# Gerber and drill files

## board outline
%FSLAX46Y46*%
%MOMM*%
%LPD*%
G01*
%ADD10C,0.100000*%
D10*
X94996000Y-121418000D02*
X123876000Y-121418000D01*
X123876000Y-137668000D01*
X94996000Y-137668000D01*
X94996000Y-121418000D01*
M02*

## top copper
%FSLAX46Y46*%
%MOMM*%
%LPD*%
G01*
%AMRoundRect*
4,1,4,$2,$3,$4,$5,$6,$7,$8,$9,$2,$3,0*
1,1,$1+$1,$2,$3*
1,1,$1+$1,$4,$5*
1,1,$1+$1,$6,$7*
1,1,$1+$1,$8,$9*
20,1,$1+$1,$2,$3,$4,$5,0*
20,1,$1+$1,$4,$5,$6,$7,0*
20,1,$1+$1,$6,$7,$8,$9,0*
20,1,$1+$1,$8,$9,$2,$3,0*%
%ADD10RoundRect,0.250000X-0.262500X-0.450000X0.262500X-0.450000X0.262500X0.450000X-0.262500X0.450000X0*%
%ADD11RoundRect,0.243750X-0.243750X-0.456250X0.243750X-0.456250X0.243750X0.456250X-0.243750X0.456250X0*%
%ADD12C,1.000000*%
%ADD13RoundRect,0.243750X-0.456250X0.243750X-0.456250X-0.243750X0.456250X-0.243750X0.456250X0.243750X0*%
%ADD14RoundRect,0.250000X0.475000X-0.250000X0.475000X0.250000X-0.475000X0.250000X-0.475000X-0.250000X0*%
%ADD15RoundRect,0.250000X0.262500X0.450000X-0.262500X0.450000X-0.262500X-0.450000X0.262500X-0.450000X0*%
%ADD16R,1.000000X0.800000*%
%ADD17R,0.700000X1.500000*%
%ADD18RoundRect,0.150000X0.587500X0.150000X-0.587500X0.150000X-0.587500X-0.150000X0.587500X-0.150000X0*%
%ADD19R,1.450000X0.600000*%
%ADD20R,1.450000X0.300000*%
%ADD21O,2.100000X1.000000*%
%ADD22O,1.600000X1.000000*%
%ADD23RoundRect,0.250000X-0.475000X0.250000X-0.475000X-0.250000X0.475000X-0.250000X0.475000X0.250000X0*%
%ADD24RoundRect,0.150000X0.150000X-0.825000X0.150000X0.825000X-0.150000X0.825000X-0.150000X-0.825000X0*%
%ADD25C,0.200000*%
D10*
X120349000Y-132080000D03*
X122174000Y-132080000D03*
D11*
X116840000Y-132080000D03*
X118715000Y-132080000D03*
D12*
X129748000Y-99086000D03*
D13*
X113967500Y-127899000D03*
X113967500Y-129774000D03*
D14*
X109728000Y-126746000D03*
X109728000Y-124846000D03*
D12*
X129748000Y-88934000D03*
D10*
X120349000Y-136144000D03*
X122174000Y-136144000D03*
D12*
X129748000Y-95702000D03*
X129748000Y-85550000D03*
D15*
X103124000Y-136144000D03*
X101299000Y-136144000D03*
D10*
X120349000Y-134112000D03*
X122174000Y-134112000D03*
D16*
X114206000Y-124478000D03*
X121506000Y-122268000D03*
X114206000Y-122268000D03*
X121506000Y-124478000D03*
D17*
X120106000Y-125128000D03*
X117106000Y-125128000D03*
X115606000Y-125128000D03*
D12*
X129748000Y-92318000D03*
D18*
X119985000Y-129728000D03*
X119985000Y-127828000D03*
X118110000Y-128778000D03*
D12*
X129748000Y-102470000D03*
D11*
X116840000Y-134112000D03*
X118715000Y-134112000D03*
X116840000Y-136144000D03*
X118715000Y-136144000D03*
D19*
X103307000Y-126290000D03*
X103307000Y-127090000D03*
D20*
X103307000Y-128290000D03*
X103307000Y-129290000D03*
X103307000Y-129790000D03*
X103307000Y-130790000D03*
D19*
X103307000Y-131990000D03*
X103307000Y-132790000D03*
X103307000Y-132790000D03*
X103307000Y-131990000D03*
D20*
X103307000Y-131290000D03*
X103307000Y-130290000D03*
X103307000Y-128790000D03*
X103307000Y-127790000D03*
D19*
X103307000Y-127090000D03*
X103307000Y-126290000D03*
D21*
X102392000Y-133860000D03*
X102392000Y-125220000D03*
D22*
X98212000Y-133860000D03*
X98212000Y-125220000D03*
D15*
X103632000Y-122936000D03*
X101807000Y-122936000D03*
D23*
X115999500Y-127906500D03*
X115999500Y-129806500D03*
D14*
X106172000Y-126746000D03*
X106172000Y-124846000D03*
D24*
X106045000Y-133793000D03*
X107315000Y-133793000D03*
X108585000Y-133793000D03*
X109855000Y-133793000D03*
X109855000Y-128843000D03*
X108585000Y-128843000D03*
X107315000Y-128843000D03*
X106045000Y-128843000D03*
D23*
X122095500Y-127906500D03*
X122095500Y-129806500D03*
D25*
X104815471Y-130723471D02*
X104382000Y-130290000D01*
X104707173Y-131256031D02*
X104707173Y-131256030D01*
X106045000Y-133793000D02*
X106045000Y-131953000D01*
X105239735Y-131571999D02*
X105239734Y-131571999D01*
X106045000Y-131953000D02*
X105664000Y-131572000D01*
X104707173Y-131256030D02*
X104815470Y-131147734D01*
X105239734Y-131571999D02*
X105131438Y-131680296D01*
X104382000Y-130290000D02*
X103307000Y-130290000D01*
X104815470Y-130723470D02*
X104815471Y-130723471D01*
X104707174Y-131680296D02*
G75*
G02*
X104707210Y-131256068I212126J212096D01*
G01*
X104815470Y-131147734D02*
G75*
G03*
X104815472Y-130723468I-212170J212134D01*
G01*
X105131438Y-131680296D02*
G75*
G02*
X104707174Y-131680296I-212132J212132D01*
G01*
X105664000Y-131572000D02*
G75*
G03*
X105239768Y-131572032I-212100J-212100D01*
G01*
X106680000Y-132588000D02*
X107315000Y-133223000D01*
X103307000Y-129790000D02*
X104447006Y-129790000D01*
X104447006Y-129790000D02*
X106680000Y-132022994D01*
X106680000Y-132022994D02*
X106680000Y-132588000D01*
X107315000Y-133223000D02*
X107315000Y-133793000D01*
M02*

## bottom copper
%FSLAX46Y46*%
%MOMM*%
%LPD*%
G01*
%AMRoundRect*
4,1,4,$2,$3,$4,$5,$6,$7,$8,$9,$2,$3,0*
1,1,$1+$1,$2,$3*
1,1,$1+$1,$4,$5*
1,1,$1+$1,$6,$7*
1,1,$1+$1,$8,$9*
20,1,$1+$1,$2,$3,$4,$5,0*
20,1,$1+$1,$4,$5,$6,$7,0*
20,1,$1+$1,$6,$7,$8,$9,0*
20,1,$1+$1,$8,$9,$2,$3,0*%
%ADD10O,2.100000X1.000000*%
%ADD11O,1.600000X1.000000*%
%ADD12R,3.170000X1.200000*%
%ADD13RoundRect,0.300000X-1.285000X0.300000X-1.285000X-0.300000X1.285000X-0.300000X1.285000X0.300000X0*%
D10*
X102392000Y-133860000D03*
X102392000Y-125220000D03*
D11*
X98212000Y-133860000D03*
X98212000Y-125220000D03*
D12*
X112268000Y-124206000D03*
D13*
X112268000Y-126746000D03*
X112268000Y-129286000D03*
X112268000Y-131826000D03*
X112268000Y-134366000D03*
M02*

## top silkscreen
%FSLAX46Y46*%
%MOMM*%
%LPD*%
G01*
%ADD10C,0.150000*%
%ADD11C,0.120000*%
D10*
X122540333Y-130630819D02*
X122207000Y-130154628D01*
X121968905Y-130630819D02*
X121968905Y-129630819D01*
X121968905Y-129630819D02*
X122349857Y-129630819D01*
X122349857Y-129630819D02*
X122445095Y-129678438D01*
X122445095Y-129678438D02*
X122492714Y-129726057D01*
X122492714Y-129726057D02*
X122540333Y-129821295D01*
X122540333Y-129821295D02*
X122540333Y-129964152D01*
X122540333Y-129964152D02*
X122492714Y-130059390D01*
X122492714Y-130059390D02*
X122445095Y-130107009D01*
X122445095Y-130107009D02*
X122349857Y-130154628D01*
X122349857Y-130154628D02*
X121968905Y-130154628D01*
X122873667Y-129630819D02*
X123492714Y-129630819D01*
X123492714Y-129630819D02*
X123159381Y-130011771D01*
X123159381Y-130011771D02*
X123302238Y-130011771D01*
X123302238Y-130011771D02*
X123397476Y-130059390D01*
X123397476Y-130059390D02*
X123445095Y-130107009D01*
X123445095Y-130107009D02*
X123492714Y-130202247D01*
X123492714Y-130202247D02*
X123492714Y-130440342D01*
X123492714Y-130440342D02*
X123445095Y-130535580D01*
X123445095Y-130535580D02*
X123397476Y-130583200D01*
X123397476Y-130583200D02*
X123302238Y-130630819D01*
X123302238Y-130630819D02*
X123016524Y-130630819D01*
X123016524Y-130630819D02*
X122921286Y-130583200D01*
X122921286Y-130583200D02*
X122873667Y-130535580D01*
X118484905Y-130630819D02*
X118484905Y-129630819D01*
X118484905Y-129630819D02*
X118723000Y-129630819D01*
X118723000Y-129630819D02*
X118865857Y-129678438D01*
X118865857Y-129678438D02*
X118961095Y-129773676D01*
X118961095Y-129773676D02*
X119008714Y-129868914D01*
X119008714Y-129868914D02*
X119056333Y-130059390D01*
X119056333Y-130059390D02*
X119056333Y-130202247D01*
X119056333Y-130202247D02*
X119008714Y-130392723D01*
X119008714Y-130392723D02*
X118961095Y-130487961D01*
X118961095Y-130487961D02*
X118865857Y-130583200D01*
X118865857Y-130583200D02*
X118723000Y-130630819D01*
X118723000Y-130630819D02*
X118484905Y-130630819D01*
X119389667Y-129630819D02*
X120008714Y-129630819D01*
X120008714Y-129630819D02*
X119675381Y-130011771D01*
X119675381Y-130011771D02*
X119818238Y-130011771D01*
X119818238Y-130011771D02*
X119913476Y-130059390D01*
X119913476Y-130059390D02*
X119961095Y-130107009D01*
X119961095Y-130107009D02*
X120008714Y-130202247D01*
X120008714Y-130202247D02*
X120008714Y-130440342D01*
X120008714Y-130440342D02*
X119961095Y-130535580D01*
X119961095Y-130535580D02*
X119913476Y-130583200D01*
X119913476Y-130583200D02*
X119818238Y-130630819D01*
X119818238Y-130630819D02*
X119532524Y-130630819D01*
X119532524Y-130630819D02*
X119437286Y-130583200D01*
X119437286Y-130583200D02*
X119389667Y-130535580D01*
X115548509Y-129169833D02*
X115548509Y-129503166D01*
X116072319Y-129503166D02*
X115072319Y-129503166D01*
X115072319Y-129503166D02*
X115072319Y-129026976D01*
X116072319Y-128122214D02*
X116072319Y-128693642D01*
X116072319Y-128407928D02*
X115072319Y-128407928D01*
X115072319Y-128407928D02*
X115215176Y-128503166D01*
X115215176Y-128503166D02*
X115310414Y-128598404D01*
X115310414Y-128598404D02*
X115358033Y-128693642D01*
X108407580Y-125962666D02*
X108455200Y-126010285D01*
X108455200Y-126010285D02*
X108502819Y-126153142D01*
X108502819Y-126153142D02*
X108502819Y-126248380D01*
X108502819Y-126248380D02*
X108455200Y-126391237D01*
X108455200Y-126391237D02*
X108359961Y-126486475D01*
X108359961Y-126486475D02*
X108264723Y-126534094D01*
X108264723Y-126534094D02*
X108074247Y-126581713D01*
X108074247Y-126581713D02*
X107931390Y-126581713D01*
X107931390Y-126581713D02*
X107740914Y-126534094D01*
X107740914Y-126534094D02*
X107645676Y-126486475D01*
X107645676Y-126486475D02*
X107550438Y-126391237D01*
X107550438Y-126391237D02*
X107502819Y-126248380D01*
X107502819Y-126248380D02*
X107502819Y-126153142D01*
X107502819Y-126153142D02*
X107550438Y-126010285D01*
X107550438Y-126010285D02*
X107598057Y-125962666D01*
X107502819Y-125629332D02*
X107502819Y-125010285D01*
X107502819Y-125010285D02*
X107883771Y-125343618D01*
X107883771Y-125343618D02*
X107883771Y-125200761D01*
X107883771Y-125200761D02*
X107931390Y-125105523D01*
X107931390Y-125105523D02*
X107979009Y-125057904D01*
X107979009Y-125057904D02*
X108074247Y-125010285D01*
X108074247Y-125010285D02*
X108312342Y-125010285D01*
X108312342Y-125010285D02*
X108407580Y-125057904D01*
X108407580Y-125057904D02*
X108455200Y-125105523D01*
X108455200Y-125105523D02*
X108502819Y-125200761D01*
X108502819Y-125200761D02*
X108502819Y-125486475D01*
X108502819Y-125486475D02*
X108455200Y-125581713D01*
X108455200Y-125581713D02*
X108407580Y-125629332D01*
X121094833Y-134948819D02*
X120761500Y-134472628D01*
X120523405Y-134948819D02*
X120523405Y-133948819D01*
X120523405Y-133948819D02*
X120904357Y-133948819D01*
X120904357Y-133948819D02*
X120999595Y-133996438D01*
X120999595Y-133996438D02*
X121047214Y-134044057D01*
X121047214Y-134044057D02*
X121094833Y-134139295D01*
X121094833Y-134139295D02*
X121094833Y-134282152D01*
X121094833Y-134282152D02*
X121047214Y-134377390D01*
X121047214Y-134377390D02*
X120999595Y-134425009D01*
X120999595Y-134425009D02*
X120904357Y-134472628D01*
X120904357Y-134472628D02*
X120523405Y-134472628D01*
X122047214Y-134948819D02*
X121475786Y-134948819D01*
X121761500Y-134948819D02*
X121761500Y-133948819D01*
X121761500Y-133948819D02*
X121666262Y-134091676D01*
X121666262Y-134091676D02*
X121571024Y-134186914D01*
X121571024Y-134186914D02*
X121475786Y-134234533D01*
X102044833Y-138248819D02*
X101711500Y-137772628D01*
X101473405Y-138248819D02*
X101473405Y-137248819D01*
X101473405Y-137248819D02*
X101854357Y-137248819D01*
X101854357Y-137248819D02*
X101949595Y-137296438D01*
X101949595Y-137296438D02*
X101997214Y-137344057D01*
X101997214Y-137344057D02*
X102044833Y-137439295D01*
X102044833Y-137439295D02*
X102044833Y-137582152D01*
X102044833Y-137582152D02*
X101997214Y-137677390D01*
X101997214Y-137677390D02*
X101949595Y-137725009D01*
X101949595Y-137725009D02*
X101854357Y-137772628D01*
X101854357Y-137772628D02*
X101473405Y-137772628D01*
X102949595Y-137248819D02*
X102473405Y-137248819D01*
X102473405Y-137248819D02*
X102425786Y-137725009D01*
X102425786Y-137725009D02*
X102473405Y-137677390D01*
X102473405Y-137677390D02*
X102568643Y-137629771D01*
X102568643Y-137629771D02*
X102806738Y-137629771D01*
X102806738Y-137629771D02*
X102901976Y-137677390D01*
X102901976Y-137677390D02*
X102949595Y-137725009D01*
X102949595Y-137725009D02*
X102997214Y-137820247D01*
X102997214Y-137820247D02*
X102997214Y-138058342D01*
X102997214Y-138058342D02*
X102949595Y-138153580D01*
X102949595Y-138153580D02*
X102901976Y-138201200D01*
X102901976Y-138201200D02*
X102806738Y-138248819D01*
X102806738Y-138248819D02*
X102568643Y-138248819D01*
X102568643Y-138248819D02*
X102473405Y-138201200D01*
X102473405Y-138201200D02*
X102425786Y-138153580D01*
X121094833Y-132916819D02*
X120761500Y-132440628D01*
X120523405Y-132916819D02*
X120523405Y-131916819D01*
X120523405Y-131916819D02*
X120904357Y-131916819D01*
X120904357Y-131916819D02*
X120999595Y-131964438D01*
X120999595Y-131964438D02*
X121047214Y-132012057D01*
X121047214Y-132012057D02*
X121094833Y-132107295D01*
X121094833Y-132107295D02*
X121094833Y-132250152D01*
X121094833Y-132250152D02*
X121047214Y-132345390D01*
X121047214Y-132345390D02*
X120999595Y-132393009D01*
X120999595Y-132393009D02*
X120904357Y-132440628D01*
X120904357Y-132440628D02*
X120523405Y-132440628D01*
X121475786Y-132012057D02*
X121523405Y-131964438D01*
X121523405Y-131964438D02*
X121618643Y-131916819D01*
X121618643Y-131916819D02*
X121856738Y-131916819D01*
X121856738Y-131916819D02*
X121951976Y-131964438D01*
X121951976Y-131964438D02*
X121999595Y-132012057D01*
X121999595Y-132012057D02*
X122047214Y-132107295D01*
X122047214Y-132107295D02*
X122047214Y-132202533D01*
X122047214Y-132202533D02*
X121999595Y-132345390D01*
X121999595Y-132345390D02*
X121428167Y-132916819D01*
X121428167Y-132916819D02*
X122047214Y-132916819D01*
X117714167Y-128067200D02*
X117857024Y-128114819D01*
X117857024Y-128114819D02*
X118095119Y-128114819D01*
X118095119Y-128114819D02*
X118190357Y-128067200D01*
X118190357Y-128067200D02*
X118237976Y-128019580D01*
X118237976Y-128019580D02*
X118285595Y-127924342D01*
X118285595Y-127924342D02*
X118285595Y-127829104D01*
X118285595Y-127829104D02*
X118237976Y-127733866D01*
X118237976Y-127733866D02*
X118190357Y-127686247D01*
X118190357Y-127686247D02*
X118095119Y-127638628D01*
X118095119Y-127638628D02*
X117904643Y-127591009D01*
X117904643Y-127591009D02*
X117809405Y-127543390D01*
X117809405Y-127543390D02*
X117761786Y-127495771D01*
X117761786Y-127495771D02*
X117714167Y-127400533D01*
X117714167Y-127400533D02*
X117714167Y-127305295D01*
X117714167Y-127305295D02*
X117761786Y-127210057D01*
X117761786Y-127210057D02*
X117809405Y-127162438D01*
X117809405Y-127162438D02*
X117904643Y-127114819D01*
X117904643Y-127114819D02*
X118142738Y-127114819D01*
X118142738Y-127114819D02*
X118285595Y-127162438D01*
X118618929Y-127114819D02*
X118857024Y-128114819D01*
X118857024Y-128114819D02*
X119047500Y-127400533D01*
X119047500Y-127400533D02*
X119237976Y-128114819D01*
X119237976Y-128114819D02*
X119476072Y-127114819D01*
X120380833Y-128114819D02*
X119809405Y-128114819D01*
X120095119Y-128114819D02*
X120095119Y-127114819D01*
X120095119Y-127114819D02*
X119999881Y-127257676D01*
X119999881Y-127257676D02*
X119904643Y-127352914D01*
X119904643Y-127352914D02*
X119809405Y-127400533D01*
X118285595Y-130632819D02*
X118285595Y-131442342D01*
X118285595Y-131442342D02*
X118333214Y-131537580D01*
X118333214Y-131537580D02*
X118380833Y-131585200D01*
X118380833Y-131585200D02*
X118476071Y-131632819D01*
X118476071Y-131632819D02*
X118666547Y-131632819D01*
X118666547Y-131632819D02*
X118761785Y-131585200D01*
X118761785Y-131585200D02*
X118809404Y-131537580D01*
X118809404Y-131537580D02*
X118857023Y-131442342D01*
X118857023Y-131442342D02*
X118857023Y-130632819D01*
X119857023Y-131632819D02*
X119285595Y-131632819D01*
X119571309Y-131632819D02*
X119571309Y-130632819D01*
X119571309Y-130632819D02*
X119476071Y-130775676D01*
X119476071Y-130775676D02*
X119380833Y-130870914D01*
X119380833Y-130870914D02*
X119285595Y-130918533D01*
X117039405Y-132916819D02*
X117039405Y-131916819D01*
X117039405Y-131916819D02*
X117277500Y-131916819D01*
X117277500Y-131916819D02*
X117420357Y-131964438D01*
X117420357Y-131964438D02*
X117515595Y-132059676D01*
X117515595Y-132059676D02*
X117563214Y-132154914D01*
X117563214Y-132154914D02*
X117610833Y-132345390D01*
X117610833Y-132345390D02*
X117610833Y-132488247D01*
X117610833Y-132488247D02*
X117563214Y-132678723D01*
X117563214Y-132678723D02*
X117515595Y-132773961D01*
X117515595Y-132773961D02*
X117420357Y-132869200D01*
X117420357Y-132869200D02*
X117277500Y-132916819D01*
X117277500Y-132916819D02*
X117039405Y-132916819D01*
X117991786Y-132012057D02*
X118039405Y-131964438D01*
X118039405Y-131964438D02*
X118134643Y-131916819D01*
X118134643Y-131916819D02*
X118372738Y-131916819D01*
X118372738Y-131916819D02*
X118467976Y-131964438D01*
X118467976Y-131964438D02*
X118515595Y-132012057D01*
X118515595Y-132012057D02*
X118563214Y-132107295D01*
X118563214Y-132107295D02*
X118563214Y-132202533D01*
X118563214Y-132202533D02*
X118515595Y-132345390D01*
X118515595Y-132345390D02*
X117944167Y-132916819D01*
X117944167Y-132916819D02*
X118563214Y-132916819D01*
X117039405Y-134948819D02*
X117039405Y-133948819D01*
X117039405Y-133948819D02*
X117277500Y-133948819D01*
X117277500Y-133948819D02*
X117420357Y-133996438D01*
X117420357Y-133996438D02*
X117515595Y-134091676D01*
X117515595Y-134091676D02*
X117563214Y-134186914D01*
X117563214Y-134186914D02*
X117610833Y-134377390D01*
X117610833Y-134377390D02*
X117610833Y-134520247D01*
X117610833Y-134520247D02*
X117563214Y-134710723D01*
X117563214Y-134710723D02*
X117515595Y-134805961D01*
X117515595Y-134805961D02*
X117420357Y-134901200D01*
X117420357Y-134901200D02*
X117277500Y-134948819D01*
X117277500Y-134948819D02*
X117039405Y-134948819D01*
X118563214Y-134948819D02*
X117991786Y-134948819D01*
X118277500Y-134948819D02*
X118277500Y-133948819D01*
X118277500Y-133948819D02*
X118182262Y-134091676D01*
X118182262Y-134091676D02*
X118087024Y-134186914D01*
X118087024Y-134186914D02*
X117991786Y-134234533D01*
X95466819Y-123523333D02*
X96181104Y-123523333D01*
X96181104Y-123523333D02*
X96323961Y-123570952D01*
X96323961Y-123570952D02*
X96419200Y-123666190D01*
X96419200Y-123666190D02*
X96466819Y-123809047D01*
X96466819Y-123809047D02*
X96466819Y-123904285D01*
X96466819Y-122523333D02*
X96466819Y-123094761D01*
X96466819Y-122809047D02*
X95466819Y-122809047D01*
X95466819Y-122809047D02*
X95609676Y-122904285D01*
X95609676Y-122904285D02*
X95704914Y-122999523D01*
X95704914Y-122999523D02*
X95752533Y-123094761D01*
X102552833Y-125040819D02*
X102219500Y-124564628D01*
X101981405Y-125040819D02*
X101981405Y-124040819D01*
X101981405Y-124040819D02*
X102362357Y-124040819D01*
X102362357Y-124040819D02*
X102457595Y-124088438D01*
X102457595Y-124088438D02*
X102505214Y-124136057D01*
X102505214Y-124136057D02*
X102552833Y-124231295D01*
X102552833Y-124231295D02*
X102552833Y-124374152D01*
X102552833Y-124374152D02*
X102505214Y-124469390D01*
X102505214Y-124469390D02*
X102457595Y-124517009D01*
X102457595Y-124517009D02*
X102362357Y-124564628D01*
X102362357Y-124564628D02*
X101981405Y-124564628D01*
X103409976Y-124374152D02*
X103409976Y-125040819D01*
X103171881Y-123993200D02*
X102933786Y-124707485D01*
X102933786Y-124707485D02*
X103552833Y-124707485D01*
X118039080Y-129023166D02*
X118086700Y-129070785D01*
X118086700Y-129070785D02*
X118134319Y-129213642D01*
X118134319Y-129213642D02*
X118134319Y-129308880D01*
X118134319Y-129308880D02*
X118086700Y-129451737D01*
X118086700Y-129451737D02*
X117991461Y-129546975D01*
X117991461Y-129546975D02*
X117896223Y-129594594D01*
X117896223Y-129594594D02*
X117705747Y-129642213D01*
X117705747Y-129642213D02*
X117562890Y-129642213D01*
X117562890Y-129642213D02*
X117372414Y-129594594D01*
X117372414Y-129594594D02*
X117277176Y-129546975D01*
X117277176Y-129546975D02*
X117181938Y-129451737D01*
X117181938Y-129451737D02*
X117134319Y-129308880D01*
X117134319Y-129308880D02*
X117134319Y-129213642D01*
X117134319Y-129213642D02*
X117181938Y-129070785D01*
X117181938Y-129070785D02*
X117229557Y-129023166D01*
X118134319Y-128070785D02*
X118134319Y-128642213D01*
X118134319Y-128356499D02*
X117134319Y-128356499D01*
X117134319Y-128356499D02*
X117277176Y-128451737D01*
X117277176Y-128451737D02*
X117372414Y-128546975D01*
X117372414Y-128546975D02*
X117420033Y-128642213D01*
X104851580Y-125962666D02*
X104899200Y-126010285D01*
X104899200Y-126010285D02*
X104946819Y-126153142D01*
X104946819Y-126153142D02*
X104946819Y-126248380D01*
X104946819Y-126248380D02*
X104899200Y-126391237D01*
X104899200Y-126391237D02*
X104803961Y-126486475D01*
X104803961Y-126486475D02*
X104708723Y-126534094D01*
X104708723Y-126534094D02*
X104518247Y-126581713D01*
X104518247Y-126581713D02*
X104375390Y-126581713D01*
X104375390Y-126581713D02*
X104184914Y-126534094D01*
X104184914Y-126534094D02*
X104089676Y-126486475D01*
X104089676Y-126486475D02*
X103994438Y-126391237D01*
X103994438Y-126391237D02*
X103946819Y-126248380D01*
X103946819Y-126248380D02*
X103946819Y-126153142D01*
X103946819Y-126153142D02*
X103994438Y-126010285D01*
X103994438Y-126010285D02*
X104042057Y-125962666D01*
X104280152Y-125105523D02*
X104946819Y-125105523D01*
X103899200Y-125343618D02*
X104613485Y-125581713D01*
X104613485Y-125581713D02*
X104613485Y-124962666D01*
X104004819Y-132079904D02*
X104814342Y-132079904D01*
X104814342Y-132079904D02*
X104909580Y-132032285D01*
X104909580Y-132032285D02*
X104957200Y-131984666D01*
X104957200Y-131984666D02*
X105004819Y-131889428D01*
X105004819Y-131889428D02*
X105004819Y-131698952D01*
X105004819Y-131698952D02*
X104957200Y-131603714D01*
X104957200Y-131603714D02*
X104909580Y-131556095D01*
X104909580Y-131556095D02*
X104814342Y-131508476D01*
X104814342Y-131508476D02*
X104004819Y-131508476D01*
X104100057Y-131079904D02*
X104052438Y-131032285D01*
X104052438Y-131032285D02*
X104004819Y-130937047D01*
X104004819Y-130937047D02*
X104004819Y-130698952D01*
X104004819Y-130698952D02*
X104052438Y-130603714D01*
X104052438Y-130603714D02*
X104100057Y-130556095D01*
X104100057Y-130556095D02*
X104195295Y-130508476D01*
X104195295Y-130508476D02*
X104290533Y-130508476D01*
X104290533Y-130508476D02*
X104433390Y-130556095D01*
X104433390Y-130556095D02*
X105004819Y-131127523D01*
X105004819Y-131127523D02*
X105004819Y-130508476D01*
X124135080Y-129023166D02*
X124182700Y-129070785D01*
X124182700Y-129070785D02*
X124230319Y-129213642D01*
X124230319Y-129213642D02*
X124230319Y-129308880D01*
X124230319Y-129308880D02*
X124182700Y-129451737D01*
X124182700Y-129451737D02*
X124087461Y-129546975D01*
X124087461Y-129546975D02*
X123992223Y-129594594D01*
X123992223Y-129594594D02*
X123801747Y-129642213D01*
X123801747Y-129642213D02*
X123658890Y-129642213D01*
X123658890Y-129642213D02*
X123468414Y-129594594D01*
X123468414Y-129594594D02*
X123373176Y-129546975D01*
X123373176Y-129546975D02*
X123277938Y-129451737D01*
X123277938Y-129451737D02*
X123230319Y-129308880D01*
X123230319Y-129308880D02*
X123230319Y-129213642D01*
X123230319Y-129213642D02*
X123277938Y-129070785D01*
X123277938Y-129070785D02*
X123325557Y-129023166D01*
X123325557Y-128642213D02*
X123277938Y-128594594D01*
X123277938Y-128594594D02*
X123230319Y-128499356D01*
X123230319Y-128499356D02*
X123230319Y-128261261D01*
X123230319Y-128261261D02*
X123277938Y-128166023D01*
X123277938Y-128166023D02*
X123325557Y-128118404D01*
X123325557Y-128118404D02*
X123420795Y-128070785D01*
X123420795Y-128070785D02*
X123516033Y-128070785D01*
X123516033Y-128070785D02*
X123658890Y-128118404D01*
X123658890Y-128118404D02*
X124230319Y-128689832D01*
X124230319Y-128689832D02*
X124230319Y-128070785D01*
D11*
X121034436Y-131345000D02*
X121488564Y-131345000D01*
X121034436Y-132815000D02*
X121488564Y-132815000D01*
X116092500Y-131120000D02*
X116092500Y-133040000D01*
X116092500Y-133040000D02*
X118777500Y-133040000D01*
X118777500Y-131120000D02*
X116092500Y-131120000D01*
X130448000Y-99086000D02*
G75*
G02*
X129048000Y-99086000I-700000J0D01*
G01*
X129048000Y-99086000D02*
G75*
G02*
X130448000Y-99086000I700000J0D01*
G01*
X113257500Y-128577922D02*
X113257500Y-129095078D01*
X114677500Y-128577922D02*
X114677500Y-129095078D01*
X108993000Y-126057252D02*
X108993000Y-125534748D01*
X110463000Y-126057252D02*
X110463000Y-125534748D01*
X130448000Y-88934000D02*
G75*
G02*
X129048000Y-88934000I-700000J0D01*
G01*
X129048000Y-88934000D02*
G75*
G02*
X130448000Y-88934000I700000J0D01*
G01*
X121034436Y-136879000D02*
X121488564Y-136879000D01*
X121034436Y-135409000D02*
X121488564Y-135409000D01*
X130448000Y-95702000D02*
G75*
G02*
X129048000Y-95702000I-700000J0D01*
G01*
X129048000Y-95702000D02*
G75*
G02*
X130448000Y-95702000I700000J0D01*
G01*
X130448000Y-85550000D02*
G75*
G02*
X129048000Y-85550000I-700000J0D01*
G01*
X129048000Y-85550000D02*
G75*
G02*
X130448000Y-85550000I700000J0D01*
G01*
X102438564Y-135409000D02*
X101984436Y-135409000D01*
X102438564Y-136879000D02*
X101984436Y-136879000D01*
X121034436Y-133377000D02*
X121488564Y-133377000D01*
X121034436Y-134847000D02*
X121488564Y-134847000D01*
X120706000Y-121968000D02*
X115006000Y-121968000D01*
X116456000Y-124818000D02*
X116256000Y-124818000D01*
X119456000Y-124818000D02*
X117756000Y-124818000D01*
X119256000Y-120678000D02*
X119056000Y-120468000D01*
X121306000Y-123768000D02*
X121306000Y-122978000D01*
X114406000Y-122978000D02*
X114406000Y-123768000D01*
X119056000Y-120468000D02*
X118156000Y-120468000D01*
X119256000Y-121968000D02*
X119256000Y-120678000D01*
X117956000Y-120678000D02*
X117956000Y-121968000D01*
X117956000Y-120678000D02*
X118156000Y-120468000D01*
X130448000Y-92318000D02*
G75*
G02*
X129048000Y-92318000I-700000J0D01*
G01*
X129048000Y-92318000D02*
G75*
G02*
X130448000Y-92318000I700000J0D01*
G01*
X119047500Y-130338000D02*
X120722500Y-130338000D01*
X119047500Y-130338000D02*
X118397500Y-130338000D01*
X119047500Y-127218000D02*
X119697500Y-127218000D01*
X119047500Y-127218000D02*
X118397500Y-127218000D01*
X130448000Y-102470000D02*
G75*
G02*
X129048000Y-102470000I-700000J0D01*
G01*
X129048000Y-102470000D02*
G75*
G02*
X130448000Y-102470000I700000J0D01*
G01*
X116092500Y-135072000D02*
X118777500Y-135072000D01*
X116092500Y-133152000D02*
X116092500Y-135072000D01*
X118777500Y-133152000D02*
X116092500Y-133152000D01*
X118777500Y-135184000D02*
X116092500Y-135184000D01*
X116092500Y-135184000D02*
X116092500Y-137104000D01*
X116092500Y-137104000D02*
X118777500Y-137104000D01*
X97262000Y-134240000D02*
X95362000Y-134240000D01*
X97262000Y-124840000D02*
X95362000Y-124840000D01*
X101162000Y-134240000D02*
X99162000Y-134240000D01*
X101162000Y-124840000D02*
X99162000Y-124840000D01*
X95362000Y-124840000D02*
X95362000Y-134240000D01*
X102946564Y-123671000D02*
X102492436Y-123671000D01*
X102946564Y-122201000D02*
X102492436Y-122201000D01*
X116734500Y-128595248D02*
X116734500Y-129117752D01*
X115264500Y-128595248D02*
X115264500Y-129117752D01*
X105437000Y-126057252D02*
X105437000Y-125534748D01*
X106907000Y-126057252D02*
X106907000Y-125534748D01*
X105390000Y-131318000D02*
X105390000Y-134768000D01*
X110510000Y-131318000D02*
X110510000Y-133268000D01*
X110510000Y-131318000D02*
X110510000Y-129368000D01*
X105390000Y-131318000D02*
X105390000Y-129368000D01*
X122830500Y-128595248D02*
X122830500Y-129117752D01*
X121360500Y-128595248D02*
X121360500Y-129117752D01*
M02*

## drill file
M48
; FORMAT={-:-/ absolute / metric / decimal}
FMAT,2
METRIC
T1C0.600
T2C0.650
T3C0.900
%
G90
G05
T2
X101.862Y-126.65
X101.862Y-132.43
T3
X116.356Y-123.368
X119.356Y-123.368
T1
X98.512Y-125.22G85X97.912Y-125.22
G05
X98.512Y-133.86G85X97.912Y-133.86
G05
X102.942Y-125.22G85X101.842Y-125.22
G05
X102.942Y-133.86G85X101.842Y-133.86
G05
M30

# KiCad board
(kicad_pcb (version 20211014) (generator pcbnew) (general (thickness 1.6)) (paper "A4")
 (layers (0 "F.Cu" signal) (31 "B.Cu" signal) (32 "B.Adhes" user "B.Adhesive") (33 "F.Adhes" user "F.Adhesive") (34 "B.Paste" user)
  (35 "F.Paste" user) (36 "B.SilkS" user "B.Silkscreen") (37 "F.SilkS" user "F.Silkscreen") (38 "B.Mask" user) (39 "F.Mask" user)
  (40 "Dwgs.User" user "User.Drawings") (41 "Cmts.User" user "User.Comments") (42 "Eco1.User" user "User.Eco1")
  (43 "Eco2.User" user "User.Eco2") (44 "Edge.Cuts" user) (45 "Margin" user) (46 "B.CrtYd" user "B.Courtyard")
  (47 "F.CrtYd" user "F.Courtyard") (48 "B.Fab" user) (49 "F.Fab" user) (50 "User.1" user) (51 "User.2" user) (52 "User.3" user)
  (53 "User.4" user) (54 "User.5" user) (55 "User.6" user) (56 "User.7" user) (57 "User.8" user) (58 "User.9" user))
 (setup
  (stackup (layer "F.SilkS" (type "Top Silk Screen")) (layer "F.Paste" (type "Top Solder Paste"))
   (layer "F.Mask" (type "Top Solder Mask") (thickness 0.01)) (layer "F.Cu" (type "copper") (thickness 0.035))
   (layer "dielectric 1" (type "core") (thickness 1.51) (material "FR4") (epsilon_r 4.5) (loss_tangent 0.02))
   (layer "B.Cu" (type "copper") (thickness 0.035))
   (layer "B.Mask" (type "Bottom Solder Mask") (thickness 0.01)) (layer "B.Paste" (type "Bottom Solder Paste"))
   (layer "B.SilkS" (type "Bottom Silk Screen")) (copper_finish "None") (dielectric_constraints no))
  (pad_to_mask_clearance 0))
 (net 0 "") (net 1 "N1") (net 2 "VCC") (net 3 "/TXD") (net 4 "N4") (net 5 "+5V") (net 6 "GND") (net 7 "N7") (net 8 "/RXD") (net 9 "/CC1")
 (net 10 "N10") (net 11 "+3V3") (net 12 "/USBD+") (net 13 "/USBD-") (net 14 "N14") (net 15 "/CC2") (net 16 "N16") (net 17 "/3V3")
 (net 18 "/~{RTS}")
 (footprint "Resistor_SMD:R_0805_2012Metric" (layer "F.Cu") (at 121.2615 132.08)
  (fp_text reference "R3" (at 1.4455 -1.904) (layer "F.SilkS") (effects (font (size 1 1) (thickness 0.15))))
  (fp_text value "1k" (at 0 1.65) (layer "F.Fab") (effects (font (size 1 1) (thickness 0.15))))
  (fp_line (start -0.227064 -0.735) (end 0.227064 -0.735) (layer "F.SilkS") (width 0.12))
  (fp_line (start -0.227064 0.735) (end 0.227064 0.735) (layer "F.SilkS") (width 0.12))
  (pad "1" smd roundrect (at -0.9125 0) (size 1.025 1.4) (layers "F.Cu" "F.Paste" "F.Mask") (roundrect_rratio 0.243902) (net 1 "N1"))
  (pad "2" smd roundrect (at 0.9125 0) (size 1.025 1.4) (layers "F.Cu" "F.Paste" "F.Mask") (roundrect_rratio 0.243902) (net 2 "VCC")))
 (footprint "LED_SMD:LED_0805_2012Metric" (layer "F.Cu") (at 117.7775 132.08)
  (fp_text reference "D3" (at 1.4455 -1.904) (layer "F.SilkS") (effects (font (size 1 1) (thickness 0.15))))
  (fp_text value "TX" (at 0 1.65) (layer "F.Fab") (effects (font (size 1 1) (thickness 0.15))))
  (fp_line (start -1.685 -0.96) (end -1.685 0.96) (layer "F.SilkS") (width 0.12))
  (fp_line (start -1.685 0.96) (end 1 0.96) (layer "F.SilkS") (width 0.12))
  (fp_line (start 1 -0.96) (end -1.685 -0.96) (layer "F.SilkS") (width 0.12))
  (pad "1" smd roundrect (at -0.9375 0) (size 0.975 1.4) (layers "F.Cu" "F.Paste" "F.Mask") (roundrect_rratio 0.25) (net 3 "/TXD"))
  (pad "2" smd roundrect (at 0.9375 0) (size 0.975 1.4) (layers "F.Cu" "F.Paste" "F.Mask") (roundrect_rratio 0.25) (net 1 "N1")))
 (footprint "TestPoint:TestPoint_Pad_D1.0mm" (layer "F.Cu") (at 129.748 99.086)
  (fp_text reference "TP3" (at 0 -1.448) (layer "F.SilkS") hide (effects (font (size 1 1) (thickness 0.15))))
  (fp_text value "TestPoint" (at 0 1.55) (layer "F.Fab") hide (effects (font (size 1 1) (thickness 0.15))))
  (fp_circle (center 0 0) (end 0 0.7) (layer "F.SilkS") (width 0.12) (fill none))
  (pad "1" smd circle (at 0 0) (size 1 1) (layers "F.Cu" "F.Mask") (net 2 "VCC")))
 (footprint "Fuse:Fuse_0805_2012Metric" (layer "F.Cu") (at 113.9675 128.8365 -90)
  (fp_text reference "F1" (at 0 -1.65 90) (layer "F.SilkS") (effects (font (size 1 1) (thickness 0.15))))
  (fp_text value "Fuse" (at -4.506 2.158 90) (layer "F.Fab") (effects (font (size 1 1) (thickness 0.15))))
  (fp_line (start -0.258578 0.71) (end 0.258578 0.71) (layer "F.SilkS") (width 0.12))
  (fp_line (start -0.258578 -0.71) (end 0.258578 -0.71) (layer "F.SilkS") (width 0.12))
  (pad "1" smd roundrect (at -0.9375 0 270) (size 0.975 1.4) (layers "F.Cu" "F.Paste" "F.Mask") (roundrect_rratio 0.25) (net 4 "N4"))
  (pad "2" smd roundrect (at 0.9375 0 270) (size 0.975 1.4) (layers "F.Cu" "F.Paste" "F.Mask") (roundrect_rratio 0.25) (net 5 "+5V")))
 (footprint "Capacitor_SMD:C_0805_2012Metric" (layer "F.Cu") (at 109.728 125.796 90)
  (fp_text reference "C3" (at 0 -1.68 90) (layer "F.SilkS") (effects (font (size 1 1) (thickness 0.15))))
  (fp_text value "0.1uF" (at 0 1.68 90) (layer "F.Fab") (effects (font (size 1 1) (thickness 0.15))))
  (fp_line (start -0.261252 -0.735) (end 0.261252 -0.735) (layer "F.SilkS") (width 0.12))
  (fp_line (start -0.261252 0.735) (end 0.261252 0.735) (layer "F.SilkS") (width 0.12))
  (pad "1" smd roundrect (at -0.95 0 90) (size 1 1.45) (layers "F.Cu" "F.Paste" "F.Mask") (roundrect_rratio 0.25) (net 2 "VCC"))
  (pad "2" smd roundrect (at 0.95 0 90) (size 1 1.45) (layers "F.Cu" "F.Paste" "F.Mask") (roundrect_rratio 0.25) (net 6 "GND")))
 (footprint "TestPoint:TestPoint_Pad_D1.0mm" (layer "F.Cu") (at 129.748 88.934)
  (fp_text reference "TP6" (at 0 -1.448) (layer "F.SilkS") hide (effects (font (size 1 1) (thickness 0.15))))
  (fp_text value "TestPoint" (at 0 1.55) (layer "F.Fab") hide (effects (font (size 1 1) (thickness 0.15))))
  (fp_circle (center 0 0) (end 0 0.7) (layer "F.SilkS") (width 0.12) (fill none))
  (pad "1" smd circle (at 0 0) (size 1 1) (layers "F.Cu" "F.Mask") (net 3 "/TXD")))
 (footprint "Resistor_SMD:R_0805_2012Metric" (layer "F.Cu") (at 121.2615 136.144)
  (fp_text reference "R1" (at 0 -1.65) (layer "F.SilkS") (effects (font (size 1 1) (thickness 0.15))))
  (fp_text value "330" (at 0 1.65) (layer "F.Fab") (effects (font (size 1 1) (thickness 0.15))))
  (fp_line (start -0.227064 0.735) (end 0.227064 0.735) (layer "F.SilkS") (width 0.12))
  (fp_line (start -0.227064 -0.735) (end 0.227064 -0.735) (layer "F.SilkS") (width 0.12))
  (pad "1" smd roundrect (at -0.9125 0) (size 1.025 1.4) (layers "F.Cu" "F.Paste" "F.Mask") (roundrect_rratio 0.243902) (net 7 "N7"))
  (pad "2" smd roundrect (at 0.9125 0) (size 1.025 1.4) (layers "F.Cu" "F.Paste" "F.Mask") (roundrect_rratio 0.243902) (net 2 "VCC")))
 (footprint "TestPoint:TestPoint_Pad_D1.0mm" (layer "F.Cu") (at 129.748 95.702)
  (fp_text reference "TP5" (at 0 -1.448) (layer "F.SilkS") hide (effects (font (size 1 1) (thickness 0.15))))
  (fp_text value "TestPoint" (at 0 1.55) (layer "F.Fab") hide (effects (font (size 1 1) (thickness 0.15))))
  (fp_circle (center 0 0) (end 0 0.7) (layer "F.SilkS") (width 0.12) (fill none))
  (pad "1" smd circle (at 0 0) (size 1 1) (layers "F.Cu" "F.Mask") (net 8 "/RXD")))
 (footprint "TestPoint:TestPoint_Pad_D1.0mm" (layer "F.Cu") (at 129.748 85.55)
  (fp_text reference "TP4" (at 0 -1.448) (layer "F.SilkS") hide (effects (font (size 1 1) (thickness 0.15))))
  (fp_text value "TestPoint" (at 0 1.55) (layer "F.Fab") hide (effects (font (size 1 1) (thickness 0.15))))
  (fp_circle (center 0 0) (end 0 0.7) (layer "F.SilkS") (width 0.12) (fill none))
  (pad "1" smd circle (at 0 0) (size 1 1) (layers "F.Cu" "F.Mask") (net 6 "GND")))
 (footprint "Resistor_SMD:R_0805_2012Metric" (layer "F.Cu") (at 102.2115 136.144 180)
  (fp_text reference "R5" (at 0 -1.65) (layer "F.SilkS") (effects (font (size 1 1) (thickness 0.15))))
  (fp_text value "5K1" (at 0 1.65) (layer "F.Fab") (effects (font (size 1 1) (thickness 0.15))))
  (fp_line (start -0.227064 0.735) (end 0.227064 0.735) (layer "F.SilkS") (width 0.12))
  (fp_line (start -0.227064 -0.735) (end 0.227064 -0.735) (layer "F.SilkS") (width 0.12))
  (pad "1" smd roundrect (at -0.9125 0 180) (size 1.025 1.4) (layers "F.Cu" "F.Paste" "F.Mask") (roundrect_rratio 0.243902) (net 6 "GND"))
  (pad "2" smd roundrect (at 0.9125 0 180) (size 1.025 1.4) (layers "F.Cu" "F.Paste" "F.Mask") (roundrect_rratio 0.243902) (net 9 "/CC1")))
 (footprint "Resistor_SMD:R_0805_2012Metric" (layer "F.Cu") (at 121.2615 134.112)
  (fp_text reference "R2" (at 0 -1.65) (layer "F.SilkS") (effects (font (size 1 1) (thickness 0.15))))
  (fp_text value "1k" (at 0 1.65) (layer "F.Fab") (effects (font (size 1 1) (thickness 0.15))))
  (fp_line (start -0.227064 -0.735) (end 0.227064 -0.735) (layer "F.SilkS") (width 0.12))
  (fp_line (start -0.227064 0.735) (end 0.227064 0.735) (layer "F.SilkS") (width 0.12))
  (pad "1" smd roundrect (at -0.9125 0) (size 1.025 1.4) (layers "F.Cu" "F.Paste" "F.Mask") (roundrect_rratio 0.243902) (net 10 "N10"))
  (pad "2" smd roundrect (at 0.9125 0) (size 1.025 1.4) (layers "F.Cu" "F.Paste" "F.Mask") (roundrect_rratio 0.243902) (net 2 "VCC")))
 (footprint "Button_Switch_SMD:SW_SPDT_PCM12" (layer "F.Cu") (at 117.856 123.698 180)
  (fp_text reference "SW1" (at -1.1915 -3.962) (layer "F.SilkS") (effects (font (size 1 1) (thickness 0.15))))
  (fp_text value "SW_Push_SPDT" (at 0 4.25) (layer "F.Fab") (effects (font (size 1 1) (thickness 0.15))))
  (fp_line (start -2.85 1.73) (end 2.85 1.73) (layer "F.SilkS") (width 0.12))
  (fp_line (start 1.4 -1.12) (end 1.6 -1.12) (layer "F.SilkS") (width 0.12))
  (fp_line (start -1.6 -1.12) (end 0.1 -1.12) (layer "F.SilkS") (width 0.12))
  (fp_line (start -1.4 3.02) (end -1.2 3.23) (layer "F.SilkS") (width 0.12))
  (fp_line (start -3.45 -0.07) (end -3.45 0.72) (layer "F.SilkS") (width 0.12))
  (fp_line (start 3.45 0.72) (end 3.45 -0.07) (layer "F.SilkS") (width 0.12))
  (fp_line (start -1.2 3.23) (end -0.3 3.23) (layer "F.SilkS") (width 0.12))
  (fp_line (start -1.4 1.73) (end -1.4 3.02) (layer "F.SilkS") (width 0.12))
  (fp_line (start -0.1 3.02) (end -0.1 1.73) (layer "F.SilkS") (width 0.12))
  (fp_line (start -0.1 3.02) (end -0.3 3.23) (layer "F.SilkS") (width 0.12))
  (pad "" smd rect (at 3.65 -0.78 180) (size 1 0.8) (layers "F.Cu" "F.Paste" "F.Mask"))
  (pad "" smd rect (at -3.65 1.43 180) (size 1 0.8) (layers "F.Cu" "F.Paste" "F.Mask"))
  (pad "" smd rect (at 3.65 1.43 180) (size 1 0.8) (layers "F.Cu" "F.Paste" "F.Mask"))
  (pad "" np_thru_hole circle (at -1.5 0.33 180) (size 0.9 0.9) (drill 0.9) (layers *.Cu *.Mask))
  (pad "" smd rect (at -3.65 -0.78 180) (size 1 0.8) (layers "F.Cu" "F.Paste" "F.Mask"))
  (pad "" np_thru_hole circle (at 1.5 0.33 180) (size 0.9 0.9) (drill 0.9) (layers *.Cu *.Mask))
  (pad "1" smd rect (at -2.25 -1.43 180) (size 0.7 1.5) (layers "F.Cu" "F.Paste" "F.Mask") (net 5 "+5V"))
  (pad "2" smd rect (at 0.75 -1.43 180) (size 0.7 1.5) (layers "F.Cu" "F.Paste" "F.Mask") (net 2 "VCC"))
  (pad "3" smd rect (at 2.25 -1.43 180) (size 0.7 1.5) (layers "F.Cu" "F.Paste" "F.Mask") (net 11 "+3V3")))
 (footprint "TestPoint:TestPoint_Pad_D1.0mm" (layer "F.Cu") (at 129.748 92.318)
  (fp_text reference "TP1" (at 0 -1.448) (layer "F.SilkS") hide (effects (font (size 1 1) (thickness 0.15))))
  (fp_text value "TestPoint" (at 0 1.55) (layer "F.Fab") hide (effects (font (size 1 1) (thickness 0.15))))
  (fp_circle (center 0 0) (end 0 0.7) (layer "F.SilkS") (width 0.12) (fill none))
  (pad "1" smd circle (at 0 0) (size 1 1) (layers "F.Cu" "F.Mask") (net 11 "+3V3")))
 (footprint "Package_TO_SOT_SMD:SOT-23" (layer "F.Cu") (at 119.0475 128.778 180)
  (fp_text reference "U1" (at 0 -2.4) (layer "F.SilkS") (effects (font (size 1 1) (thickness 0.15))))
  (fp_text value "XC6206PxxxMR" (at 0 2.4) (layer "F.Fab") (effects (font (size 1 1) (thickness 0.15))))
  (fp_line (start 0 -1.56) (end -1.675 -1.56) (layer "F.SilkS") (width 0.12))
  (fp_line (start 0 -1.56) (end 0.65 -1.56) (layer "F.SilkS") (width 0.12))
  (fp_line (start 0 1.56) (end -0.65 1.56) (layer "F.SilkS") (width 0.12))
  (fp_line (start 0 1.56) (end 0.65 1.56) (layer "F.SilkS") (width 0.12))
  (pad "1" smd roundrect (at -0.9375 -0.95 180) (size 1.475 0.6) (layers "F.Cu" "F.Paste" "F.Mask") (roundrect_rratio 0.25) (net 6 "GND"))
  (pad "2" smd roundrect (at -0.9375 0.95 180) (size 1.475 0.6) (layers "F.Cu" "F.Paste" "F.Mask") (roundrect_rratio 0.25) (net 11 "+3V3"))
  (pad "3" smd roundrect (at 0.9375 0 180) (size 1.475 0.6) (layers "F.Cu" "F.Paste" "F.Mask") (roundrect_rratio 0.25) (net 5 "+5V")))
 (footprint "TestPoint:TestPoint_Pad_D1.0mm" (layer "F.Cu") (at 129.748 102.47)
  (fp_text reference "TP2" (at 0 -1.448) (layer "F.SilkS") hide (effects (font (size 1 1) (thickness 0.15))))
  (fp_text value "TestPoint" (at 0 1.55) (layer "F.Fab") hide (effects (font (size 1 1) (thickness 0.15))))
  (fp_circle (center 0 0) (end 0 0.7) (layer "F.SilkS") (width 0.12) (fill none))
  (pad "1" smd circle (at 0 0) (size 1 1) (layers "F.Cu" "F.Mask") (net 5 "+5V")))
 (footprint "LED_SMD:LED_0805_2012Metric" (layer "F.Cu") (at 117.7775 134.112)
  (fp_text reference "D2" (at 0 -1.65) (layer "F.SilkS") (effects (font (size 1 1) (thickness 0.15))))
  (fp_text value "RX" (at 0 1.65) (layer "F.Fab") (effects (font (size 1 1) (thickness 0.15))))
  (fp_line (start -1.685 0.96) (end 1 0.96) (layer "F.SilkS") (width 0.12))
  (fp_line (start -1.685 -0.96) (end -1.685 0.96) (layer "F.SilkS") (width 0.12))
  (fp_line (start 1 -0.96) (end -1.685 -0.96) (layer "F.SilkS") (width 0.12))
  (pad "1" smd roundrect (at -0.9375 0) (size 0.975 1.4) (layers "F.Cu" "F.Paste" "F.Mask") (roundrect_rratio 0.25) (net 8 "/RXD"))
  (pad "2" smd roundrect (at 0.9375 0) (size 0.975 1.4) (layers "F.Cu" "F.Paste" "F.Mask") (roundrect_rratio 0.25) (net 10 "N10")))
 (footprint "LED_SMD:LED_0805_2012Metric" (layer "F.Cu") (at 117.7775 136.144)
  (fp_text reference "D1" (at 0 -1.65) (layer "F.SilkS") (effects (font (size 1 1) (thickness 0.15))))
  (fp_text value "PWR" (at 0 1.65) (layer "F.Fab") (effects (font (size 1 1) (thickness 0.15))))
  (fp_line (start 1 -0.96) (end -1.685 -0.96) (layer "F.SilkS") (width 0.12))
  (fp_line (start -1.685 -0.96) (end -1.685 0.96) (layer "F.SilkS") (width 0.12))
  (fp_line (start -1.685 0.96) (end 1 0.96) (layer "F.SilkS") (width 0.12))
  (pad "1" smd roundrect (at -0.9375 0) (size 0.975 1.4) (layers "F.Cu" "F.Paste" "F.Mask") (roundrect_rratio 0.25) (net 6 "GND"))
  (pad "2" smd roundrect (at 0.9375 0) (size 0.975 1.4) (layers "F.Cu" "F.Paste" "F.Mask") (roundrect_rratio 0.25) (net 7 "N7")))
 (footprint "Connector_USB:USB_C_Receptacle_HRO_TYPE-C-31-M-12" (layer "F.Cu") (at 99.262 129.54 -90)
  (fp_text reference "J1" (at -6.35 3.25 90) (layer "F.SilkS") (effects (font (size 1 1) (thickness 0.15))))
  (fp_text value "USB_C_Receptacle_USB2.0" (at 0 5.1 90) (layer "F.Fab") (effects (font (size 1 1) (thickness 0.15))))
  (fp_line (start 4.7 2) (end 4.7 3.9) (layer "F.SilkS") (width 0.12))
  (fp_line (start -4.7 2) (end -4.7 3.9) (layer "F.SilkS") (width 0.12))
  (fp_line (start 4.7 -1.9) (end 4.7 0.1) (layer "F.SilkS") (width 0.12))
  (fp_line (start -4.7 -1.9) (end -4.7 0.1) (layer "F.SilkS") (width 0.12))
  (fp_line (start -4.7 3.9) (end 4.7 3.9) (layer "F.SilkS") (width 0.12))
  (pad "" np_thru_hole circle (at 2.89 -2.6 270) (size 0.65 0.65) (drill 0.65) (layers *.Cu *.Mask))
  (pad "" np_thru_hole circle (at -2.89 -2.6 270) (size 0.65 0.65) (drill 0.65) (layers *.Cu *.Mask))
  (pad "A1" smd rect (at -3.25 -4.045 270) (size 0.6 1.45) (layers "F.Cu" "F.Paste" "F.Mask") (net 6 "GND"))
  (pad "A4" smd rect (at -2.45 -4.045 270) (size 0.6 1.45) (layers "F.Cu" "F.Paste" "F.Mask") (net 4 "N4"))
  (pad "A5" smd rect (at -1.25 -4.045 270) (size 0.3 1.45) (layers "F.Cu" "F.Paste" "F.Mask") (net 9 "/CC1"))
  (pad "A6" smd rect (at -0.25 -4.045 270) (size 0.3 1.45) (layers "F.Cu" "F.Paste" "F.Mask") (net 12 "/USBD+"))
  (pad "A7" smd rect (at 0.25 -4.045 270) (size 0.3 1.45) (layers "F.Cu" "F.Paste" "F.Mask") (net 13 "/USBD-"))
  (pad "A8" smd rect (at 1.25 -4.045 270) (size 0.3 1.45) (layers "F.Cu" "F.Paste" "F.Mask") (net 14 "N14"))
  (pad "A9" smd rect (at 2.45 -4.045 270) (size 0.6 1.45) (layers "F.Cu" "F.Paste" "F.Mask") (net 4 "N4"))
  (pad "A12" smd rect (at 3.25 -4.045 270) (size 0.6 1.45) (layers "F.Cu" "F.Paste" "F.Mask") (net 6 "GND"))
  (pad "B1" smd rect (at 3.25 -4.045 270) (size 0.6 1.45) (layers "F.Cu" "F.Paste" "F.Mask") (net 6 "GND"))
  (pad "B4" smd rect (at 2.45 -4.045 270) (size 0.6 1.45) (layers "F.Cu" "F.Paste" "F.Mask") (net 4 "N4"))
  (pad "B5" smd rect (at 1.75 -4.045 270) (size 0.3 1.45) (layers "F.Cu" "F.Paste" "F.Mask") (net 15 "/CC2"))
  (pad "B6" smd rect (at 0.75 -4.045 270) (size 0.3 1.45) (layers "F.Cu" "F.Paste" "F.Mask") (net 12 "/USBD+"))
  (pad "B7" smd rect (at -0.75 -4.045 270) (size 0.3 1.45) (layers "F.Cu" "F.Paste" "F.Mask") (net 13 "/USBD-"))
  (pad "B8" smd rect (at -1.75 -4.045 270) (size 0.3 1.45) (layers "F.Cu" "F.Paste" "F.Mask") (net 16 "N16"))
  (pad "B9" smd rect (at -2.45 -4.045 270) (size 0.6 1.45) (layers "F.Cu" "F.Paste" "F.Mask") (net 4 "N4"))
  (pad "B12" smd rect (at -3.25 -4.045 270) (size 0.6 1.45) (layers "F.Cu" "F.Paste" "F.Mask") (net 6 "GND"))
  (pad "S1" thru_hole oval (at 4.32 -3.13 270) (size 1 2.1) (drill oval 0.6 1.7) (layers *.Cu *.Mask) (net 6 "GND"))
  (pad "S1" thru_hole oval (at -4.32 -3.13 270) (size 1 2.1) (drill oval 0.6 1.7) (layers *.Cu *.Mask) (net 6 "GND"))
  (pad "S1" thru_hole oval (at 4.32 1.05 270) (size 1 1.6) (drill oval 0.6 1.2) (layers *.Cu *.Mask) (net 6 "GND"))
  (pad "S1" thru_hole oval (at -4.32 1.05 270) (size 1 1.6) (drill oval 0.6 1.2) (layers *.Cu *.Mask) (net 6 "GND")))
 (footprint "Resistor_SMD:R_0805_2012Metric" (layer "F.Cu") (at 102.7195 122.936 180)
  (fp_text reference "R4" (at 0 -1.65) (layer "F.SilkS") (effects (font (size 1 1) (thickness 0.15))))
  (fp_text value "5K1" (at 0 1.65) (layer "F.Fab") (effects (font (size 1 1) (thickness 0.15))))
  (fp_line (start -0.227064 -0.735) (end 0.227064 -0.735) (layer "F.SilkS") (width 0.12))
  (fp_line (start -0.227064 0.735) (end 0.227064 0.735) (layer "F.SilkS") (width 0.12))
  (pad "1" smd roundrect (at -0.9125 0 180) (size 1.025 1.4) (layers "F.Cu" "F.Paste" "F.Mask") (roundrect_rratio 0.243902) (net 6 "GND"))
  (pad "2" smd roundrect (at 0.9125 0 180) (size 1.025 1.4) (layers "F.Cu" "F.Paste" "F.Mask") (roundrect_rratio 0.243902) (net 15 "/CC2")))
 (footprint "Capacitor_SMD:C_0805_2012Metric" (layer "F.Cu") (at 115.9995 128.8565 -90)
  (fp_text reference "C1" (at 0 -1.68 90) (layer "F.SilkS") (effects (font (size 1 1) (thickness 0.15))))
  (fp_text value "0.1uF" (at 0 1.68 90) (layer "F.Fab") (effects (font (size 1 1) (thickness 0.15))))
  (fp_line (start -0.261252 -0.735) (end 0.261252 -0.735) (layer "F.SilkS") (width 0.12))
  (fp_line (start -0.261252 0.735) (end 0.261252 0.735) (layer "F.SilkS") (width 0.12))
  (pad "1" smd roundrect (at -0.95 0 270) (size 1 1.45) (layers "F.Cu" "F.Paste" "F.Mask") (roundrect_rratio 0.25) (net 5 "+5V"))
  (pad "2" smd roundrect (at 0.95 0 270) (size 1 1.45) (layers "F.Cu" "F.Paste" "F.Mask") (roundrect_rratio 0.25) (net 6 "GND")))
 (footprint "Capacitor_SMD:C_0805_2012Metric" (layer "F.Cu") (at 106.172 125.796 90)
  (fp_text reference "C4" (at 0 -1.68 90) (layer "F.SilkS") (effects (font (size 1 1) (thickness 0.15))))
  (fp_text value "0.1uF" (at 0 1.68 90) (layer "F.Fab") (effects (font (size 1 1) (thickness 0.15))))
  (fp_line (start -0.261252 -0.735) (end 0.261252 -0.735) (layer "F.SilkS") (width 0.12))
  (fp_line (start -0.261252 0.735) (end 0.261252 0.735) (layer "F.SilkS") (width 0.12))
  (pad "1" smd roundrect (at -0.95 0 90) (size 1 1.45) (layers "F.Cu" "F.Paste" "F.Mask") (roundrect_rratio 0.25) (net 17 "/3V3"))
  (pad "2" smd roundrect (at 0.95 0 90) (size 1 1.45) (layers "F.Cu" "F.Paste" "F.Mask") (roundrect_rratio 0.25) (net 6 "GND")))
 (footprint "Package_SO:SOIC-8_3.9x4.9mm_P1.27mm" (layer "F.Cu") (at 107.95 131.318 90)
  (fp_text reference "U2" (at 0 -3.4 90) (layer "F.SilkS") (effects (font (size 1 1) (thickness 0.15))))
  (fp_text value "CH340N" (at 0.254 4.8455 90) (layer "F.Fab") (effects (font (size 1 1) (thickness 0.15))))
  (fp_line (start 0 -2.56) (end -3.45 -2.56) (layer "F.SilkS") (width 0.12))
  (fp_line (start 0 2.56) (end -1.95 2.56) (layer "F.SilkS") (width 0.12))
  (fp_line (start 0 2.56) (end 1.95 2.56) (layer "F.SilkS") (width 0.12))
  (fp_line (start 0 -2.56) (end 1.95 -2.56) (layer "F.SilkS") (width 0.12))
  (pad "1" smd roundrect (at -2.475 -1.905 90) (size 1.95 0.6) (layers "F.Cu" "F.Paste" "F.Mask") (roundrect_rratio 0.25) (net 12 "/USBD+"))
  (pad "2" smd roundrect (at -2.475 -0.635 90) (size 1.95 0.6) (layers "F.Cu" "F.Paste" "F.Mask") (roundrect_rratio 0.25) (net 13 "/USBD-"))
  (pad "3" smd roundrect (at -2.475 0.635 90) (size 1.95 0.6) (layers "F.Cu" "F.Paste" "F.Mask") (roundrect_rratio 0.25) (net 6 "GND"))
  (pad "4" smd roundrect (at -2.475 1.905 90) (size 1.95 0.6) (layers "F.Cu" "F.Paste" "F.Mask") (roundrect_rratio 0.25) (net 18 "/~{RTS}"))
  (pad "5" smd roundrect (at 2.475 1.905 90) (size 1.95 0.6) (layers "F.Cu" "F.Paste" "F.Mask") (roundrect_rratio 0.25) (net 2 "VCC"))
  (pad "6" smd roundrect (at 2.475 0.635 90) (size 1.95 0.6) (layers "F.Cu" "F.Paste" "F.Mask") (roundrect_rratio 0.25) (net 3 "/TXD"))
  (pad "7" smd roundrect (at 2.475 -0.635 90) (size 1.95 0.6) (layers "F.Cu" "F.Paste" "F.Mask") (roundrect_rratio 0.25) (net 8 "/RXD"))
  (pad "8" smd roundrect (at 2.475 -1.905 90) (size 1.95 0.6) (layers "F.Cu" "F.Paste" "F.Mask") (roundrect_rratio 0.25) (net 17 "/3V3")))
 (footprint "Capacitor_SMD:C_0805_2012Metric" (layer "F.Cu") (at 122.0955 128.8565 -90)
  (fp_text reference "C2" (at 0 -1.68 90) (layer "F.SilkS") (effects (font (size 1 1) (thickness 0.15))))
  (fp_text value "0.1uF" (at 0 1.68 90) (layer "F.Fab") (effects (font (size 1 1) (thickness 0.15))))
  (fp_line (start -0.261252 -0.735) (end 0.261252 -0.735) (layer "F.SilkS") (width 0.12))
  (fp_line (start -0.261252 0.735) (end 0.261252 0.735) (layer "F.SilkS") (width 0.12))
  (pad "1" smd roundrect (at -0.95 0 270) (size 1 1.45) (layers "F.Cu" "F.Paste" "F.Mask") (roundrect_rratio 0.25) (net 11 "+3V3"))
  (pad "2" smd roundrect (at 0.95 0 270) (size 1 1.45) (layers "F.Cu" "F.Paste" "F.Mask") (roundrect_rratio 0.25) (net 6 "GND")))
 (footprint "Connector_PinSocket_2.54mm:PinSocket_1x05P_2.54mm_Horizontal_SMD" (layer "B.Cu") (at 112.268 124.206 180)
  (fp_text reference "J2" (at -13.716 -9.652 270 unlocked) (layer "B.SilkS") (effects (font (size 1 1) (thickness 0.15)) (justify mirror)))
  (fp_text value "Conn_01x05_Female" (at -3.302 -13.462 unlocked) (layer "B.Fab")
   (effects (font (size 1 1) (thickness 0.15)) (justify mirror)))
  (pad "1" smd rect (at 0 0 270) (size 1.2 3.17) (layers "B.Cu" "B.Paste" "B.Mask") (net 6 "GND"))
  (pad "2" smd roundrect (at 0 -2.54 270) (size 1.2 3.17) (layers "B.Cu" "B.Paste" "B.Mask") (roundrect_rratio 0.25) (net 18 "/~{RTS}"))
  (pad "3" smd roundrect (at 0 -5.08 270) (size 1.2 3.17) (layers "B.Cu" "B.Paste" "B.Mask") (roundrect_rratio 0.25) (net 3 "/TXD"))
  (pad "4" smd roundrect (at 0 -7.62 270) (size 1.2 3.17) (layers "B.Cu" "B.Paste" "B.Mask") (roundrect_rratio 0.25) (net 8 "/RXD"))
  (pad "5" smd roundrect (at 0 -10.16 270) (size 1.2 3.17) (layers "B.Cu" "B.Paste" "B.Mask") (roundrect_rratio 0.25) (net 2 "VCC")))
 (gr_rect (start 94.996 121.418) (end 123.876 137.668) (layer "Edge.Cuts") (width 0.1) (fill none))
 (segment (start 104.815471 130.723471) (end 104.382 130.29) (width 0.2) (layer "F.Cu") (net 12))
 (segment (start 104.707173 131.256031) (end 104.707173 131.25603) (width 0.2) (layer "F.Cu") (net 12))
 (segment (start 106.045 133.793) (end 106.045 131.953) (width 0.2) (layer "F.Cu") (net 12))
 (segment (start 105.239735 131.571999) (end 105.239734 131.571999) (width 0.2) (layer "F.Cu") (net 12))
 (segment (start 106.045 131.953) (end 105.664 131.572) (width 0.2) (layer "F.Cu") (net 12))
 (segment (start 104.707173 131.25603) (end 104.81547 131.147734) (width 0.2) (layer "F.Cu") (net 12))
 (segment (start 105.239734 131.571999) (end 105.131438 131.680296) (width 0.2) (layer "F.Cu") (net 12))
 (segment (start 104.382 130.29) (end 103.307 130.29) (width 0.2) (layer "F.Cu") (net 12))
 (segment (start 104.81547 130.72347) (end 104.815471 130.723471) (width 0.2) (layer "F.Cu") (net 12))
 (arc (start 104.707174 131.680296) (mid 104.619304 131.468163) (end 104.707173 131.256031) (width 0.2) (layer "F.Cu") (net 12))
 (arc (start 104.81547 131.147734) (mid 104.903338 130.935602) (end 104.81547 130.72347) (width 0.2) (layer "F.Cu") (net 12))
 (arc (start 105.131438 131.680296) (mid 104.919306 131.768164) (end 104.707174 131.680296) (width 0.2) (layer "F.Cu") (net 12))
 (arc (start 105.664 131.572) (mid 105.451867 131.48413) (end 105.239735 131.571999) (width 0.2) (layer "F.Cu") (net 12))
 (segment (start 106.68 132.588) (end 107.315 133.223) (width 0.2) (layer "F.Cu") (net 13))
 (segment (start 103.307 129.79) (end 104.447006 129.79) (width 0.2) (layer "F.Cu") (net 13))
 (segment (start 104.447006 129.79) (end 106.68 132.022994) (width 0.2) (layer "F.Cu") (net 13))
 (segment (start 106.68 132.022994) (end 106.68 132.588) (width 0.2) (layer "F.Cu") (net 13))
 (segment (start 107.315 133.223) (end 107.315 133.793) (width 0.2) (layer "F.Cu") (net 13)))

